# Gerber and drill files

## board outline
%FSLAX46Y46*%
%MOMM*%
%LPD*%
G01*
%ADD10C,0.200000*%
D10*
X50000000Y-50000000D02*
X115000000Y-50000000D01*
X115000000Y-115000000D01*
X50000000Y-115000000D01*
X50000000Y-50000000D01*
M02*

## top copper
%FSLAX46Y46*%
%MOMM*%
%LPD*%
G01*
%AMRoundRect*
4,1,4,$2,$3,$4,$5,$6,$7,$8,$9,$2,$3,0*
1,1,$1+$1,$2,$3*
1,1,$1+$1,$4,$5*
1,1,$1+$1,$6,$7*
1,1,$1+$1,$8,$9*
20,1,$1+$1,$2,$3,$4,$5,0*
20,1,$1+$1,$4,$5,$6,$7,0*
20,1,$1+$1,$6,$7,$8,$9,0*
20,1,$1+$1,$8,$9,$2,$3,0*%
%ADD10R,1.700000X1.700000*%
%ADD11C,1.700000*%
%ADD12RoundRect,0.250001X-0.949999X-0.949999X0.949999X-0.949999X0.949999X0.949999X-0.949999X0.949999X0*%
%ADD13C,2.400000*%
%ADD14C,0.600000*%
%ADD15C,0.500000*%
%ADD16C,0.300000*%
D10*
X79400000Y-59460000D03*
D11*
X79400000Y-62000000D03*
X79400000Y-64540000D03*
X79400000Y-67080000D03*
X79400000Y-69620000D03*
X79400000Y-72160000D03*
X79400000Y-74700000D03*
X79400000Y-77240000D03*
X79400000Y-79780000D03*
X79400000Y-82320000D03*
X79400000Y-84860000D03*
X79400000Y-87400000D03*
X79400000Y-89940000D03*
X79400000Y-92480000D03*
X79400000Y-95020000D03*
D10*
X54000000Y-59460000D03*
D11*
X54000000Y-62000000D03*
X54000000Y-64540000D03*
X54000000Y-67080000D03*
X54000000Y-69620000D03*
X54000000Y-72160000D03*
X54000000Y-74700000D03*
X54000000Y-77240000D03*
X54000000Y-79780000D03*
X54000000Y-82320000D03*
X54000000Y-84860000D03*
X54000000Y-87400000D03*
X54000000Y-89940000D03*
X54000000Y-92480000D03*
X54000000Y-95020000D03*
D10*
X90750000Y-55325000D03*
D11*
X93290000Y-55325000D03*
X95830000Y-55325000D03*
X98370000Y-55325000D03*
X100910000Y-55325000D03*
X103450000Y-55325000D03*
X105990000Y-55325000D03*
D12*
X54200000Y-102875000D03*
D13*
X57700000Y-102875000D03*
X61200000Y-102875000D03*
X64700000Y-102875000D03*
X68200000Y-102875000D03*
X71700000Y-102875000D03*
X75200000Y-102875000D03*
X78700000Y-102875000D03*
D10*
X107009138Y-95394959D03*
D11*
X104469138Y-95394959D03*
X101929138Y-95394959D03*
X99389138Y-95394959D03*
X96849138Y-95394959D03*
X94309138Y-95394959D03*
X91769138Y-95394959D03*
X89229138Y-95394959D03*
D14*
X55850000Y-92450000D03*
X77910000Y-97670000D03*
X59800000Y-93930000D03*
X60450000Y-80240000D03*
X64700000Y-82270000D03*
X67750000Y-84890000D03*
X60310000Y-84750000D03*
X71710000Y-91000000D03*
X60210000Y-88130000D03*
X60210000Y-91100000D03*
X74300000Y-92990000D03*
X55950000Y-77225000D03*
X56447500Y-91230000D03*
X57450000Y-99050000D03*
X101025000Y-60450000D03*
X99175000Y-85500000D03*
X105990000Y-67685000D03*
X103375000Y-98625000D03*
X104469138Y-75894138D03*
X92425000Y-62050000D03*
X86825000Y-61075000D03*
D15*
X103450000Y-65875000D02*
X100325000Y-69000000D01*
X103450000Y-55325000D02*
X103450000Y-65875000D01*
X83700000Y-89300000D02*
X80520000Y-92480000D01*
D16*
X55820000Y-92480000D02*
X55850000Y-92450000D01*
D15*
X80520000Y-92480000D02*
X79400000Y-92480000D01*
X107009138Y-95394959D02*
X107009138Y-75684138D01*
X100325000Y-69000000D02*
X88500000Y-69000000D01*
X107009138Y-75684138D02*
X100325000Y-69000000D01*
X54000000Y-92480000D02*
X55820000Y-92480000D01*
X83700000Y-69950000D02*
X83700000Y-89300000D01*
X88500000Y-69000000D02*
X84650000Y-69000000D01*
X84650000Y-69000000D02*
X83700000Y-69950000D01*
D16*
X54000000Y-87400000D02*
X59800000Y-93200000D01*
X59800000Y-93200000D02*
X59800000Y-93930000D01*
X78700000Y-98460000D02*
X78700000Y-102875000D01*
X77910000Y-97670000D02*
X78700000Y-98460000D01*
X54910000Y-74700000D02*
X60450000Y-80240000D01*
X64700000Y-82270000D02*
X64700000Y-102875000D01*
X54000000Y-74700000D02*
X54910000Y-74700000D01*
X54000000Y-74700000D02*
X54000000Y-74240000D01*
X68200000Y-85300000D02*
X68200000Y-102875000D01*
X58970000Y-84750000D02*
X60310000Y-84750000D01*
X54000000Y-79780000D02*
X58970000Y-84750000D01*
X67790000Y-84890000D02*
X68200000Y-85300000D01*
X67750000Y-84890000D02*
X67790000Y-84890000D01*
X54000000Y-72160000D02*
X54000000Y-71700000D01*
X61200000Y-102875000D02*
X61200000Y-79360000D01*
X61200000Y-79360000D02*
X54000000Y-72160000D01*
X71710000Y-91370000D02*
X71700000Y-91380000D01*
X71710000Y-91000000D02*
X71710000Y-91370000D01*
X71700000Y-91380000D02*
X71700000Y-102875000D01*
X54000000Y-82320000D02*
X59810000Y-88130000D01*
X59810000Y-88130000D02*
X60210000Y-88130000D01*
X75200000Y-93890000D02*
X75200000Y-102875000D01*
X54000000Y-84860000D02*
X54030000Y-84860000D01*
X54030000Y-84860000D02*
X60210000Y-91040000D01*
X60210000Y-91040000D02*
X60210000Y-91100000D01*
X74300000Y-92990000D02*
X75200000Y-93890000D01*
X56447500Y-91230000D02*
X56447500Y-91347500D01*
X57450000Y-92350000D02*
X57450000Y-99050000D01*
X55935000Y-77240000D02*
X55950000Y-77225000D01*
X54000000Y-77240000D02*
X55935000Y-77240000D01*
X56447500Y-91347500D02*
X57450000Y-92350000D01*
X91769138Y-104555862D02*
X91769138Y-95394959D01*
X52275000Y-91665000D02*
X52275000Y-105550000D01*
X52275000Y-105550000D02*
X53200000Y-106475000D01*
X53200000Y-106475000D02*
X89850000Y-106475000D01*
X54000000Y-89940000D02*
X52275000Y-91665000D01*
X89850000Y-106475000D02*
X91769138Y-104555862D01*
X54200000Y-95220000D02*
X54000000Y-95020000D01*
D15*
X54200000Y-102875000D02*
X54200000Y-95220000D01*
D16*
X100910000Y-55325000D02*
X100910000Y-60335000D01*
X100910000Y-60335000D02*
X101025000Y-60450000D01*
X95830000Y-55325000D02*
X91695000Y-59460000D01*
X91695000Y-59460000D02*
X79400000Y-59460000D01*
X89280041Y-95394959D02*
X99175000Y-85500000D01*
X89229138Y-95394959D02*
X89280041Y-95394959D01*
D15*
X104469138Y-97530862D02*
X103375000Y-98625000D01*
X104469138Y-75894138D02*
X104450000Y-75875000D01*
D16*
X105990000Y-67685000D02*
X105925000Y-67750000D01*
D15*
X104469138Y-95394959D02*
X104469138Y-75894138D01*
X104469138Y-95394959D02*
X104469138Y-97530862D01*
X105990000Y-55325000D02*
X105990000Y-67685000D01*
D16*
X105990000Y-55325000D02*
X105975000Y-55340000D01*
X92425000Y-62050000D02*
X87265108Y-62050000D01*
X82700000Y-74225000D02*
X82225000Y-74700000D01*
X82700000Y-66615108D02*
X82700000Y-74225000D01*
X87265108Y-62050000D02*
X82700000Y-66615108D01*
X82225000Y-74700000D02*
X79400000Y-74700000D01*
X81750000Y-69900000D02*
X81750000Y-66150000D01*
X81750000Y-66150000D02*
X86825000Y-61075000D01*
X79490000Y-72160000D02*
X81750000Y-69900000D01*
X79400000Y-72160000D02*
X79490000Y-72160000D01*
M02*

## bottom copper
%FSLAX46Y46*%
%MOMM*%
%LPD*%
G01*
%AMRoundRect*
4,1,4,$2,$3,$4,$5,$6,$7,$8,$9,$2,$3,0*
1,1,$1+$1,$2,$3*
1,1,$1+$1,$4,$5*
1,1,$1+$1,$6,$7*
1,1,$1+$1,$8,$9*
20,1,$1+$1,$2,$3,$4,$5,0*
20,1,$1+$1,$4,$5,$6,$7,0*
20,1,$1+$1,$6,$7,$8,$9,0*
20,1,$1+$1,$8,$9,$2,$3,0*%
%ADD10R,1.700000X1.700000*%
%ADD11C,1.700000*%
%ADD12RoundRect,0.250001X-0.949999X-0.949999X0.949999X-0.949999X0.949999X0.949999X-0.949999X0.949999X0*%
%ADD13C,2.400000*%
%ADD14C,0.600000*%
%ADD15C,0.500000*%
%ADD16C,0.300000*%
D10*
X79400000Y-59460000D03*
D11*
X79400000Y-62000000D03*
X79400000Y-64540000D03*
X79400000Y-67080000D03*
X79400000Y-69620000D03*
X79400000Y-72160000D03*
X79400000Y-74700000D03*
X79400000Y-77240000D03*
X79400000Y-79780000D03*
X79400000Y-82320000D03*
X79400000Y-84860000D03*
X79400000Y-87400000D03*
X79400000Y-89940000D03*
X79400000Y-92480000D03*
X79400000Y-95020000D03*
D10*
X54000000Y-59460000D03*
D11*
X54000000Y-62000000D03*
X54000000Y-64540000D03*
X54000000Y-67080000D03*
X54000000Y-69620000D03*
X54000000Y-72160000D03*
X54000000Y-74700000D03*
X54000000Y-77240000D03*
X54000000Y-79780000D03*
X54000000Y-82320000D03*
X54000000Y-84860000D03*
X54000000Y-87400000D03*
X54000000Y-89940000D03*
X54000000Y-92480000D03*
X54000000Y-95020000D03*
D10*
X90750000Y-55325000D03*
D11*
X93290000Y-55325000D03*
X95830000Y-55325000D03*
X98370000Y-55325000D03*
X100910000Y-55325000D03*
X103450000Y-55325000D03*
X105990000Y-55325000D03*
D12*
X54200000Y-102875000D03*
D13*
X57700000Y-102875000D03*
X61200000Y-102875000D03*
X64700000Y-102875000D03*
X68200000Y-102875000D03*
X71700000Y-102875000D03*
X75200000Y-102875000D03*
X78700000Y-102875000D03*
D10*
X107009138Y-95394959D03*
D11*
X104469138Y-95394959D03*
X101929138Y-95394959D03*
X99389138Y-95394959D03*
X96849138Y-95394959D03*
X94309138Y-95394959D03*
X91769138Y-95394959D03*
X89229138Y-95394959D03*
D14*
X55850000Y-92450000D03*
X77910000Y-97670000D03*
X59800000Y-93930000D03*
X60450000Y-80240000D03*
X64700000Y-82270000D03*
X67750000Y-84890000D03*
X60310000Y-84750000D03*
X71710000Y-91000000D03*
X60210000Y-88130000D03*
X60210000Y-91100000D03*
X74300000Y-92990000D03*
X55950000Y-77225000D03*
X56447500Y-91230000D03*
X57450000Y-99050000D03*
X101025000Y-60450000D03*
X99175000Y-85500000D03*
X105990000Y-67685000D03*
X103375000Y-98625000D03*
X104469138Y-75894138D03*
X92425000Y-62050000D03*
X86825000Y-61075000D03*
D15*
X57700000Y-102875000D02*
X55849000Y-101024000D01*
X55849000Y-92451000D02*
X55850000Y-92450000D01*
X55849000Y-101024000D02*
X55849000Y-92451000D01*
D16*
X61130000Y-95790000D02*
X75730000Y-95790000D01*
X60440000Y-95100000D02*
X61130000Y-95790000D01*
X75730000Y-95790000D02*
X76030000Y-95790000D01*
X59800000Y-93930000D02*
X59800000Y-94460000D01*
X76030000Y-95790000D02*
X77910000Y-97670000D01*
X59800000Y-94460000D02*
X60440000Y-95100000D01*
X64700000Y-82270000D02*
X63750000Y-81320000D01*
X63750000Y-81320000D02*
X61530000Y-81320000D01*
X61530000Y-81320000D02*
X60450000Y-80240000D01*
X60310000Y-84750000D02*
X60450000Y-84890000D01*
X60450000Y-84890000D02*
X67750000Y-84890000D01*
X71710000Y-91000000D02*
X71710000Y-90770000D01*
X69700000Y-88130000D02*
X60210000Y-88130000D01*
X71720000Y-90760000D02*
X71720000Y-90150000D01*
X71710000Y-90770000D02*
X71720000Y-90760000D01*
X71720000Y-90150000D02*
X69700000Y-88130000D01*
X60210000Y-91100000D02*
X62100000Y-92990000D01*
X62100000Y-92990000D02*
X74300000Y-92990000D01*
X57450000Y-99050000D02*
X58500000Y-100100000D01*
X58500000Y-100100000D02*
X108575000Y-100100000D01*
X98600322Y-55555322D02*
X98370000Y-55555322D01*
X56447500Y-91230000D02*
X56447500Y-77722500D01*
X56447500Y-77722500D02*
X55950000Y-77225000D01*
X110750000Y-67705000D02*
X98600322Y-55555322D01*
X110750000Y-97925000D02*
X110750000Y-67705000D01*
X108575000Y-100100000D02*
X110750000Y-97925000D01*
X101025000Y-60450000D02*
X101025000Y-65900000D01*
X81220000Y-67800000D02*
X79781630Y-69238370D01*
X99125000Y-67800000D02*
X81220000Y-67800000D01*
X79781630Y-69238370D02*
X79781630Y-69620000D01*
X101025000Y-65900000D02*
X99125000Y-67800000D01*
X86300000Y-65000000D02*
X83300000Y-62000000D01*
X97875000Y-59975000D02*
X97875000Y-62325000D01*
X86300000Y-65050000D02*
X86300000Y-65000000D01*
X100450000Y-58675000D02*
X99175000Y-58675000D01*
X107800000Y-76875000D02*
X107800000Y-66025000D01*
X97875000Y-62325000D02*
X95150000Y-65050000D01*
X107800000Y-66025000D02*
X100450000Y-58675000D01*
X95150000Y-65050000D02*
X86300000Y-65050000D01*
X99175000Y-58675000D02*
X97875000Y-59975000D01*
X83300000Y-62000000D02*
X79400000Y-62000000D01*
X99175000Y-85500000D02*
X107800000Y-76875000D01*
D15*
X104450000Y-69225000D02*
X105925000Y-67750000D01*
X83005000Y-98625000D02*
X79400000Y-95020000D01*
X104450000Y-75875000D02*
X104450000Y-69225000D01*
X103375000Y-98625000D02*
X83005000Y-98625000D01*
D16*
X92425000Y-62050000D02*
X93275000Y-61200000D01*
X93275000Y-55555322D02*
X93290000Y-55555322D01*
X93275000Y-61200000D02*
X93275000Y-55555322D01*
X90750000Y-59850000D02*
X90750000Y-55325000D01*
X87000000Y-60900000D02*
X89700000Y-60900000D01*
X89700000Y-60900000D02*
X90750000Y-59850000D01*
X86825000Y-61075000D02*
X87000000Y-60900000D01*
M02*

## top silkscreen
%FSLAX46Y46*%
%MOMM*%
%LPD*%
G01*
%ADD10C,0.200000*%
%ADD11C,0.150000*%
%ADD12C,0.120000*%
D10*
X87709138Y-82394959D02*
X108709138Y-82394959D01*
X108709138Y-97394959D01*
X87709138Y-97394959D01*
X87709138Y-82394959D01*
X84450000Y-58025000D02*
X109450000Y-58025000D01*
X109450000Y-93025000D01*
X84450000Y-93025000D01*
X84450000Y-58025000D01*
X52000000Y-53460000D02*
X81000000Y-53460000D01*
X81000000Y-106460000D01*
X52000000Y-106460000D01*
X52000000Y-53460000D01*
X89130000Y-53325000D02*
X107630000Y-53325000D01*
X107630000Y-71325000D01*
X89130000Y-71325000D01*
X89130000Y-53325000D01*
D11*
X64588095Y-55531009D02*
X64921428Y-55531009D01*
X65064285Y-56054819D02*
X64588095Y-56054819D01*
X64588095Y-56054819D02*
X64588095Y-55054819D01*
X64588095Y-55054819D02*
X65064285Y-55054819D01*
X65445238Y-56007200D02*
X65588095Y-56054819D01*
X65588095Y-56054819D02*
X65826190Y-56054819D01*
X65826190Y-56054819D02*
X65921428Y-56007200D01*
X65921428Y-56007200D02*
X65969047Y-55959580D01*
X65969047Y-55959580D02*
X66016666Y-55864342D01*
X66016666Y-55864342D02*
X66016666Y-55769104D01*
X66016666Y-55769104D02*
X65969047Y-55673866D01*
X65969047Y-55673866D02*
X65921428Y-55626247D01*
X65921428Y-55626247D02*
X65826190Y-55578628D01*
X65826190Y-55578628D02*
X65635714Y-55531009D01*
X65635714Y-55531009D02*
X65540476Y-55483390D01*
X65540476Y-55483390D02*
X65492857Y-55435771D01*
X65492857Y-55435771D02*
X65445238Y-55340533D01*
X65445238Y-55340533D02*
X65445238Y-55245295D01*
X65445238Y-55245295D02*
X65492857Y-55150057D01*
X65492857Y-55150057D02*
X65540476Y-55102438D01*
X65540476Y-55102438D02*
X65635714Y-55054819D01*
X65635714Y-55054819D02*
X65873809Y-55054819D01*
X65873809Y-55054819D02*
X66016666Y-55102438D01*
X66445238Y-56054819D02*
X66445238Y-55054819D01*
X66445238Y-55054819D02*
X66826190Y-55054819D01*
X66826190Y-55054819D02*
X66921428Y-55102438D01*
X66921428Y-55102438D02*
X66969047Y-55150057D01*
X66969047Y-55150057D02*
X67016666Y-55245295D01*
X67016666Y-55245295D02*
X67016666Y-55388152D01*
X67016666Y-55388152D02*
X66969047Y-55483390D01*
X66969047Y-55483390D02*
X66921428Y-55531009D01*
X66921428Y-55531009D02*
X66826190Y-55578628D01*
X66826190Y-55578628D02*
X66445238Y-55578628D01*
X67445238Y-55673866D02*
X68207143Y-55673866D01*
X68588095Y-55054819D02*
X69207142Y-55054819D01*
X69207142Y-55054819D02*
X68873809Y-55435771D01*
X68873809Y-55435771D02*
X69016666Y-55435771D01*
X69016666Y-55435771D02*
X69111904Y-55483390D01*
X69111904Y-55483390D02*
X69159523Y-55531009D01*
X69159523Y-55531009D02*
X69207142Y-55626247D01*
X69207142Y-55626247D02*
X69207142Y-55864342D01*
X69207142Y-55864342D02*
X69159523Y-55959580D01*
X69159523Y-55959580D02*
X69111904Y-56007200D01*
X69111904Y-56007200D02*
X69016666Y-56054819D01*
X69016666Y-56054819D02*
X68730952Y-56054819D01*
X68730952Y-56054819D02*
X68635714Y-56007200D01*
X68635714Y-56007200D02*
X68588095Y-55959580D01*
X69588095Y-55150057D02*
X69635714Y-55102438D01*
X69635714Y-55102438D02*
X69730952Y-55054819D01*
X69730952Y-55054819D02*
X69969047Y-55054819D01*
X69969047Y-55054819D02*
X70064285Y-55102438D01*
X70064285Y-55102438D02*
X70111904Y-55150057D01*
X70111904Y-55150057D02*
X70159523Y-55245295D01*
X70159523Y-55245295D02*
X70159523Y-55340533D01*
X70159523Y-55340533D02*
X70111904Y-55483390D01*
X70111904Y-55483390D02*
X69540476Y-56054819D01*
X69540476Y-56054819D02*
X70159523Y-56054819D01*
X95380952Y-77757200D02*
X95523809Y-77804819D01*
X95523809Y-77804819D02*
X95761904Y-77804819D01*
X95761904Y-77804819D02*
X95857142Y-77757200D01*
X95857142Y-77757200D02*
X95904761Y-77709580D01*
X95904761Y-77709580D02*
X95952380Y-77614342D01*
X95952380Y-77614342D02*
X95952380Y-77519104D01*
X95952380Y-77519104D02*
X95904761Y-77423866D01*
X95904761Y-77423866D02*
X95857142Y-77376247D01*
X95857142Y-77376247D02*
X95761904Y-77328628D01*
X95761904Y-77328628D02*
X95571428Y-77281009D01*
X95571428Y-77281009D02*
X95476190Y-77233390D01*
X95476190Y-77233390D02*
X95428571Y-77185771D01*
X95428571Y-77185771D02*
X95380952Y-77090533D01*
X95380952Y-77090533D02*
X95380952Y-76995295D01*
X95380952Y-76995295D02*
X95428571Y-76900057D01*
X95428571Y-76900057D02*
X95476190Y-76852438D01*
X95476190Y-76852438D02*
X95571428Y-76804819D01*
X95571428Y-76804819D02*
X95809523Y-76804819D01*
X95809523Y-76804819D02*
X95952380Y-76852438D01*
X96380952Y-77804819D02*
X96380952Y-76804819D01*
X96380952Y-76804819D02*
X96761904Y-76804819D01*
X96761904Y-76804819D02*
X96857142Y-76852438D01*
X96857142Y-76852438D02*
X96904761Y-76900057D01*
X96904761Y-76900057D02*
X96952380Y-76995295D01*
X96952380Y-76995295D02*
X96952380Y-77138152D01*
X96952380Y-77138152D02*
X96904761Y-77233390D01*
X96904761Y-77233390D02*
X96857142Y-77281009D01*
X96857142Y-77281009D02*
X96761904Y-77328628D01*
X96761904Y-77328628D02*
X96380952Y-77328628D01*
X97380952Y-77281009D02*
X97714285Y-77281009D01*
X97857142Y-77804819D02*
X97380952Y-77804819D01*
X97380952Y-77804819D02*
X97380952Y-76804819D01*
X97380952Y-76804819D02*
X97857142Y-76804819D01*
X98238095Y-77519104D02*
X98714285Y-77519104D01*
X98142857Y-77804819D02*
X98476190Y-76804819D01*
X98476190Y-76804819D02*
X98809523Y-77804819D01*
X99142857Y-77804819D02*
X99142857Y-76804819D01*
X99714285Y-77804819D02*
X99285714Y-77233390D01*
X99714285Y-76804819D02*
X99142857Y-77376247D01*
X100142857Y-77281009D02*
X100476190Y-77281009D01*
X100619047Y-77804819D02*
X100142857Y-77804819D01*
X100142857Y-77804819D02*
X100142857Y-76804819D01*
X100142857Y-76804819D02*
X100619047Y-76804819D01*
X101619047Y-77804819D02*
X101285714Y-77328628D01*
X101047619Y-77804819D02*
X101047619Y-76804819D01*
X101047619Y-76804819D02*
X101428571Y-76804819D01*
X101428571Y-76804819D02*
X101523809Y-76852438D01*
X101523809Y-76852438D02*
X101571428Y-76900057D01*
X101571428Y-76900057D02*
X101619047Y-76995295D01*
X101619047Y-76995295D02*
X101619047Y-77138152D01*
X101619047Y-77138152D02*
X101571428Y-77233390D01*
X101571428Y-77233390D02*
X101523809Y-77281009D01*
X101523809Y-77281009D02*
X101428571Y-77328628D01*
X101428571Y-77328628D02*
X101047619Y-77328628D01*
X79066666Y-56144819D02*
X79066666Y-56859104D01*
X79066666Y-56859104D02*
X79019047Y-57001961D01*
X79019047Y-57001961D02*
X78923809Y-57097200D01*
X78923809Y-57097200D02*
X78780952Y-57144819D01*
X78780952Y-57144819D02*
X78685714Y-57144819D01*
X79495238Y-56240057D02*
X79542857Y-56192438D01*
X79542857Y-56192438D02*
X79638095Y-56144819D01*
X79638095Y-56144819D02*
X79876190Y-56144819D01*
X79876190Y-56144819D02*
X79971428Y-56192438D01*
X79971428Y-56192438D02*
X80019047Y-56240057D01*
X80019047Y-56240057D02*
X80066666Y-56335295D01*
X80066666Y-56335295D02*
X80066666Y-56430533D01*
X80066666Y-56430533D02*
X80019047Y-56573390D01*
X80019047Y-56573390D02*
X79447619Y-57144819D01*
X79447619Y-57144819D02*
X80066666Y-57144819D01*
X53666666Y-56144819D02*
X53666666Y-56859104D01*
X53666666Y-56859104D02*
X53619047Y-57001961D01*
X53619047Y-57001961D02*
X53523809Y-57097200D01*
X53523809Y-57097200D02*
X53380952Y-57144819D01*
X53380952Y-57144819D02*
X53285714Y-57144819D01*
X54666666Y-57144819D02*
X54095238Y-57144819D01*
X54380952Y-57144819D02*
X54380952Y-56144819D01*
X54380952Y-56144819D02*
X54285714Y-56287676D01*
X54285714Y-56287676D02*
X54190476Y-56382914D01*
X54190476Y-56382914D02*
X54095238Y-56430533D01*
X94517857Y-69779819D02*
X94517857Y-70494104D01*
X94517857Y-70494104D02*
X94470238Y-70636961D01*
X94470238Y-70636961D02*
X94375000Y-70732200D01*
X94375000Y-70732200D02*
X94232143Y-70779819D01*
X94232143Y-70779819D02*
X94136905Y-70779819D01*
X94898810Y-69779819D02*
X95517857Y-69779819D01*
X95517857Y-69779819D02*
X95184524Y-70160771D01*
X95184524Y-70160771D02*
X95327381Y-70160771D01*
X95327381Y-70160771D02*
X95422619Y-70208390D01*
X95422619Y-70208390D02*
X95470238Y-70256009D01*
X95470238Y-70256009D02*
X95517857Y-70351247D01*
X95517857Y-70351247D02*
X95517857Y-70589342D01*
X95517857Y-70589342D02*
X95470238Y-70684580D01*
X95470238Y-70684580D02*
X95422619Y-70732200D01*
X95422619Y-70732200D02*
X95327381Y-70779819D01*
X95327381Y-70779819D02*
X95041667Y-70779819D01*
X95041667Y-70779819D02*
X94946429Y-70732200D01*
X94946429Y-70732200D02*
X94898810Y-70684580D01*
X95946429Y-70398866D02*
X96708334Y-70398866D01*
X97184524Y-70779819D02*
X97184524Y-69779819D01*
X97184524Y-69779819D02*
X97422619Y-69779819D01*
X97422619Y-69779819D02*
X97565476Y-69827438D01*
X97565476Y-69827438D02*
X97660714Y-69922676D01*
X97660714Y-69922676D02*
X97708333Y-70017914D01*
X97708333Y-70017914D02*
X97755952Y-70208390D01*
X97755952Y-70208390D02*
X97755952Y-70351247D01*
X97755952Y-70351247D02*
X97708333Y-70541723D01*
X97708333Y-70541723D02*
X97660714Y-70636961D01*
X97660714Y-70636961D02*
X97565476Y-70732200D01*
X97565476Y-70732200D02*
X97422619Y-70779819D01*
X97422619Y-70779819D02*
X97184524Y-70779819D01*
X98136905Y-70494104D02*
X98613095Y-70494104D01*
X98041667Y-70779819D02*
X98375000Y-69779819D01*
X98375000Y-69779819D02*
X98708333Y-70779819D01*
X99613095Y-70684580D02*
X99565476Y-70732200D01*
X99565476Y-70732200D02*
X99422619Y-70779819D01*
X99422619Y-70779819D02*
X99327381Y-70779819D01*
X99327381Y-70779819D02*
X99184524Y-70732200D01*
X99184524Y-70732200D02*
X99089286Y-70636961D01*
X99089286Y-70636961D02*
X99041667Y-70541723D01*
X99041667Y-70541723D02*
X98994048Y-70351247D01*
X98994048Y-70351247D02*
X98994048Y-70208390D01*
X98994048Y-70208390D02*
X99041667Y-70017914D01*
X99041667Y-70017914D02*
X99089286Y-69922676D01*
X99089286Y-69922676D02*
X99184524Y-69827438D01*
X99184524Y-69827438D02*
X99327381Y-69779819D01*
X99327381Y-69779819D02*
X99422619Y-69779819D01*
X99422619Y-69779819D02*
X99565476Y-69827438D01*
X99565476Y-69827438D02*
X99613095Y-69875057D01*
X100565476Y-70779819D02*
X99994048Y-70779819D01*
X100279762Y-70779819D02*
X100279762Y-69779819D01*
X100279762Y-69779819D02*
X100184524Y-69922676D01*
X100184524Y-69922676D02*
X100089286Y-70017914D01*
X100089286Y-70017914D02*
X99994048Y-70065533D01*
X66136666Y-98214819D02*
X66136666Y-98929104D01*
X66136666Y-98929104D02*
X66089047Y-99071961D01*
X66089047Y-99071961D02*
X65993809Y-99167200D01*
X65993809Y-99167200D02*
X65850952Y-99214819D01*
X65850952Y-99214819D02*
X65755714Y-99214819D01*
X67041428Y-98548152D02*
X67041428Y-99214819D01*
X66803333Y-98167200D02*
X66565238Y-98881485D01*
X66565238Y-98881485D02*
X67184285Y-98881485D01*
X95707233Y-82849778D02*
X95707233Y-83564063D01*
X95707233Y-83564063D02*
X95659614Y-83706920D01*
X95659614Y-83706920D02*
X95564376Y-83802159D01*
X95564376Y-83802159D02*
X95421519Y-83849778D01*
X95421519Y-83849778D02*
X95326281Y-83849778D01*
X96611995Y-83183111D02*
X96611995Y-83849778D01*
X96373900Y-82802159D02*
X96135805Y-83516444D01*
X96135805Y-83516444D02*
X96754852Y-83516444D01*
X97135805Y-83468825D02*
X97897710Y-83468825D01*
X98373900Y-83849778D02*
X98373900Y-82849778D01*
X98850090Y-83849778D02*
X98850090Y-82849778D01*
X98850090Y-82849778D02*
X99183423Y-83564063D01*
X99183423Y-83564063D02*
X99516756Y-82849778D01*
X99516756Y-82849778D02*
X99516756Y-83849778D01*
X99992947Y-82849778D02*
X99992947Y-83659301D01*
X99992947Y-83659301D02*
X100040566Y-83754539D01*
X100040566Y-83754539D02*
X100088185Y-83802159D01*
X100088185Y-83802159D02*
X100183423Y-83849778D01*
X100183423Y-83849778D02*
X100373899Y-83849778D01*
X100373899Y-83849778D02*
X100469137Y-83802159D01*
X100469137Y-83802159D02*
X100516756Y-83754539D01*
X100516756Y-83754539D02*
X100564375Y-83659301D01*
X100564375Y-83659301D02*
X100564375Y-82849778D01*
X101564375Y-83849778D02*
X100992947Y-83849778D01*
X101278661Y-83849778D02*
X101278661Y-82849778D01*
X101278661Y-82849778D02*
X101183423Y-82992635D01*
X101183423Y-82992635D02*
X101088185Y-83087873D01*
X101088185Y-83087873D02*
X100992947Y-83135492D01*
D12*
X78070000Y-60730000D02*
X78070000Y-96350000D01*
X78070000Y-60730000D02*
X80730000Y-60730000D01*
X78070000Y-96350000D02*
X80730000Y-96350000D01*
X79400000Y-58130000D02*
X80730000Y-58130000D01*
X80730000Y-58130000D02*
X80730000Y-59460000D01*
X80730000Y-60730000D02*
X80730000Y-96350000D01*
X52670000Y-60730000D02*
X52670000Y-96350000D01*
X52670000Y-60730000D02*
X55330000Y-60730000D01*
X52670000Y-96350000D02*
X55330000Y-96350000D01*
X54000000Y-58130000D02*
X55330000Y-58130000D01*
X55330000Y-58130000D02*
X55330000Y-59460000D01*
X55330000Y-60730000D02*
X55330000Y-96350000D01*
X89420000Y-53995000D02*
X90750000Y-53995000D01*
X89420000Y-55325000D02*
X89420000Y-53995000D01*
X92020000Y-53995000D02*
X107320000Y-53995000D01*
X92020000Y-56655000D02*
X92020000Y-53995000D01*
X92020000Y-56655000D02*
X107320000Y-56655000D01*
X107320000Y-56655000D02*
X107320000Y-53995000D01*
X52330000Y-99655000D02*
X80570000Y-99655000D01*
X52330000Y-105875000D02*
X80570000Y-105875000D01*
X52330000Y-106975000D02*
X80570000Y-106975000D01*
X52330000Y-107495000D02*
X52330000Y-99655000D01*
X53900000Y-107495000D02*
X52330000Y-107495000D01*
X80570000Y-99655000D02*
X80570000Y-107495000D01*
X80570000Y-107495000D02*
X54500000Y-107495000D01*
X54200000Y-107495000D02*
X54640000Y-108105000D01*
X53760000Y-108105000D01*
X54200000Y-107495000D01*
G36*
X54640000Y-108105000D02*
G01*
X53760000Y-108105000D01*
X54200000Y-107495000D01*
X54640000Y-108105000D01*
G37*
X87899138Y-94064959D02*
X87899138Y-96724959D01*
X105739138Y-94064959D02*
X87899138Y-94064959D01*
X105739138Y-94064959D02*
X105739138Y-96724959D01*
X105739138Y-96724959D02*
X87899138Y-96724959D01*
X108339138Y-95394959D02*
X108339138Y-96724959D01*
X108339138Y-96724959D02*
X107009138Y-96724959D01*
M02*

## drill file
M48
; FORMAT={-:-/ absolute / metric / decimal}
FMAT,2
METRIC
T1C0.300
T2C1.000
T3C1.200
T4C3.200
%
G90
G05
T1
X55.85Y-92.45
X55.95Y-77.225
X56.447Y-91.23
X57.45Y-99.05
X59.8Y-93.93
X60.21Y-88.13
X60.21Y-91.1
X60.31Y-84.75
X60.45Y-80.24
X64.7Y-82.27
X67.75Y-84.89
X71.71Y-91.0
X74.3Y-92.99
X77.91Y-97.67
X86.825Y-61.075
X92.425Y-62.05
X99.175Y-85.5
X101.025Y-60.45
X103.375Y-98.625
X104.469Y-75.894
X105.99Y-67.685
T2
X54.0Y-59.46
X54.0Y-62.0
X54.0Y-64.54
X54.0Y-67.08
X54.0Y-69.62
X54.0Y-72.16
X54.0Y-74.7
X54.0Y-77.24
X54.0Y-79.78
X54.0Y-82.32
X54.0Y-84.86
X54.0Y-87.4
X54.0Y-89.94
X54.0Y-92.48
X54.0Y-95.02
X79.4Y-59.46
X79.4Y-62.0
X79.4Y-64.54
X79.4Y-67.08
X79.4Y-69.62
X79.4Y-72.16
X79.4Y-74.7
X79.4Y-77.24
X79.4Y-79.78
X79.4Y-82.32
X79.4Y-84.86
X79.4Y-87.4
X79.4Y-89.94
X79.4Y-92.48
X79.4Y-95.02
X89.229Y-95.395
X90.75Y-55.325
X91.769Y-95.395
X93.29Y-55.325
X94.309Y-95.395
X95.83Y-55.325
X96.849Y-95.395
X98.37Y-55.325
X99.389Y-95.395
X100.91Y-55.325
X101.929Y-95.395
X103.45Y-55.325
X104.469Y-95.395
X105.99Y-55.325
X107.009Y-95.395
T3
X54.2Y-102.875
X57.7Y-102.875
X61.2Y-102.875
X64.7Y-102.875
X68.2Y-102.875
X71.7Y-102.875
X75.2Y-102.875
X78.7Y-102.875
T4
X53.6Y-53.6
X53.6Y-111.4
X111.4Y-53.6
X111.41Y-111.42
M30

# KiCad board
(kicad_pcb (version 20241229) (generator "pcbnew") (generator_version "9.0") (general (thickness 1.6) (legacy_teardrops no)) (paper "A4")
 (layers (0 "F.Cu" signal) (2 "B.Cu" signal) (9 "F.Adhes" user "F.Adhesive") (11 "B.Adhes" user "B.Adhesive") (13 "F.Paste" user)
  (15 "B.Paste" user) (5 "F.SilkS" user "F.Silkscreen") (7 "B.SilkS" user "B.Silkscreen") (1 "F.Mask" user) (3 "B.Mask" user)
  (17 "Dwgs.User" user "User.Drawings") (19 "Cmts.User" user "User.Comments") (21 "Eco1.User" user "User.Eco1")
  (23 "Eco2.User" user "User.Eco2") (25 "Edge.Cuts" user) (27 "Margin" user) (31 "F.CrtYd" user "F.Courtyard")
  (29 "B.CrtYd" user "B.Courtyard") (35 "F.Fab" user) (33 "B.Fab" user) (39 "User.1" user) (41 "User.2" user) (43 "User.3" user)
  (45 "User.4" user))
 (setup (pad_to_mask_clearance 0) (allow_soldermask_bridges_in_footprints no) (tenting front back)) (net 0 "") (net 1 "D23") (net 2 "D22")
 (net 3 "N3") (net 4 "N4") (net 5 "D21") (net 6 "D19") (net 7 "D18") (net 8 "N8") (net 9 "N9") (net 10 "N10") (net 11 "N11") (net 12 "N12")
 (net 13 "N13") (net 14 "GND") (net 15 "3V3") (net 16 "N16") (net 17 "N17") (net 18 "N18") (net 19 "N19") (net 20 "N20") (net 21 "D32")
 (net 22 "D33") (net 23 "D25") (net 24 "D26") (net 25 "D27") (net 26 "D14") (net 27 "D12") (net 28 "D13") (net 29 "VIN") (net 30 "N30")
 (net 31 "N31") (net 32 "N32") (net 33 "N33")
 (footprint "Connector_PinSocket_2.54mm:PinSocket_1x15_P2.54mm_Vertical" (layer "F.Cu") (at 79.4 59.46)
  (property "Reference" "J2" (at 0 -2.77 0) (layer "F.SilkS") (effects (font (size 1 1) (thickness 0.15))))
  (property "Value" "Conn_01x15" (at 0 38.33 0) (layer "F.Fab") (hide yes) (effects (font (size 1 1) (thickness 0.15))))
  (fp_line (start -1.33 1.27) (end -1.33 36.89) (stroke (width 0.12) (type solid)) (layer "F.SilkS"))
  (fp_line (start -1.33 1.27) (end 1.33 1.27) (stroke (width 0.12) (type solid)) (layer "F.SilkS"))
  (fp_line (start -1.33 36.89) (end 1.33 36.89) (stroke (width 0.12) (type solid)) (layer "F.SilkS"))
  (fp_line (start 0 -1.33) (end 1.33 -1.33) (stroke (width 0.12) (type solid)) (layer "F.SilkS"))
  (fp_line (start 1.33 -1.33) (end 1.33 0) (stroke (width 0.12) (type solid)) (layer "F.SilkS"))
  (fp_line (start 1.33 1.27) (end 1.33 36.89) (stroke (width 0.12) (type solid)) (layer "F.SilkS"))
  (pad "1" thru_hole rect (at 0 0) (size 1.7 1.7) (drill 1) (layers "*.Cu" "*.Mask") (remove_unused_layers no) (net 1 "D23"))
  (pad "2" thru_hole circle (at 0 2.54) (size 1.7 1.7) (drill 1) (layers "*.Cu" "*.Mask") (remove_unused_layers no) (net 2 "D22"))
  (pad "3" thru_hole circle (at 0 5.08) (size 1.7 1.7) (drill 1) (layers "*.Cu" "*.Mask") (remove_unused_layers no) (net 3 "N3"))
  (pad "4" thru_hole circle (at 0 7.62) (size 1.7 1.7) (drill 1) (layers "*.Cu" "*.Mask") (remove_unused_layers no) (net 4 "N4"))
  (pad "5" thru_hole circle (at 0 10.16) (size 1.7 1.7) (drill 1) (layers "*.Cu" "*.Mask") (remove_unused_layers no) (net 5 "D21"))
  (pad "6" thru_hole circle (at 0 12.7) (size 1.7 1.7) (drill 1) (layers "*.Cu" "*.Mask") (remove_unused_layers no) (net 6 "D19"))
  (pad "7" thru_hole circle (at 0 15.24) (size 1.7 1.7) (drill 1) (layers "*.Cu" "*.Mask") (remove_unused_layers no) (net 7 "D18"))
  (pad "8" thru_hole circle (at 0 17.78) (size 1.7 1.7) (drill 1) (layers "*.Cu" "*.Mask") (remove_unused_layers no) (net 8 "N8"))
  (pad "9" thru_hole circle (at 0 20.32) (size 1.7 1.7) (drill 1) (layers "*.Cu" "*.Mask") (remove_unused_layers no) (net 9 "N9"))
  (pad "10" thru_hole circle (at 0 22.86) (size 1.7 1.7) (drill 1) (layers "*.Cu" "*.Mask") (remove_unused_layers no) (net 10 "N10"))
  (pad "11" thru_hole circle (at 0 25.4) (size 1.7 1.7) (drill 1) (layers "*.Cu" "*.Mask") (remove_unused_layers no) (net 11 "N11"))
  (pad "12" thru_hole circle (at 0 27.94) (size 1.7 1.7) (drill 1) (layers "*.Cu" "*.Mask") (remove_unused_layers no) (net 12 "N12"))
  (pad "13" thru_hole circle (at 0 30.48) (size 1.7 1.7) (drill 1) (layers "*.Cu" "*.Mask") (remove_unused_layers no) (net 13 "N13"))
  (pad "14" thru_hole circle (at 0 33.02) (size 1.7 1.7) (drill 1) (layers "*.Cu" "*.Mask") (remove_unused_layers no) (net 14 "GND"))
  (pad "15" thru_hole circle (at 0 35.56) (size 1.7 1.7) (drill 1) (layers "*.Cu" "*.Mask") (remove_unused_layers no) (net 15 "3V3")))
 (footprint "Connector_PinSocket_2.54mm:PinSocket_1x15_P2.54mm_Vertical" (layer "F.Cu") (at 54 59.46)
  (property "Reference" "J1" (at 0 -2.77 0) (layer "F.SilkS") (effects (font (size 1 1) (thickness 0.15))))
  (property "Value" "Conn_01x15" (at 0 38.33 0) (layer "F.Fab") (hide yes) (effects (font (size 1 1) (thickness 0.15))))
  (fp_line (start -1.33 1.27) (end -1.33 36.89) (stroke (width 0.12) (type solid)) (layer "F.SilkS"))
  (fp_line (start -1.33 1.27) (end 1.33 1.27) (stroke (width 0.12) (type solid)) (layer "F.SilkS"))
  (fp_line (start -1.33 36.89) (end 1.33 36.89) (stroke (width 0.12) (type solid)) (layer "F.SilkS"))
  (fp_line (start 0 -1.33) (end 1.33 -1.33) (stroke (width 0.12) (type solid)) (layer "F.SilkS"))
  (fp_line (start 1.33 -1.33) (end 1.33 0) (stroke (width 0.12) (type solid)) (layer "F.SilkS"))
  (fp_line (start 1.33 1.27) (end 1.33 36.89) (stroke (width 0.12) (type solid)) (layer "F.SilkS"))
  (pad "1" thru_hole rect (at 0 0) (size 1.7 1.7) (drill 1) (layers "*.Cu" "*.Mask") (remove_unused_layers no) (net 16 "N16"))
  (pad "2" thru_hole circle (at 0 2.54) (size 1.7 1.7) (drill 1) (layers "*.Cu" "*.Mask") (remove_unused_layers no) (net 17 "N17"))
  (pad "3" thru_hole circle (at 0 5.08) (size 1.7 1.7) (drill 1) (layers "*.Cu" "*.Mask") (remove_unused_layers no) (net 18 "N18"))
  (pad "4" thru_hole circle (at 0 7.62) (size 1.7 1.7) (drill 1) (layers "*.Cu" "*.Mask") (remove_unused_layers no) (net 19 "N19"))
  (pad "5" thru_hole circle (at 0 10.16) (size 1.7 1.7) (drill 1) (layers "*.Cu" "*.Mask") (remove_unused_layers no) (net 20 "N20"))
  (pad "6" thru_hole circle (at 0 12.7) (size 1.7 1.7) (drill 1) (layers "*.Cu" "*.Mask") (remove_unused_layers no) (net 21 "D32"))
  (pad "7" thru_hole circle (at 0 15.24) (size 1.7 1.7) (drill 1) (layers "*.Cu" "*.Mask") (remove_unused_layers no) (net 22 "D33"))
  (pad "8" thru_hole circle (at 0 17.78) (size 1.7 1.7) (drill 1) (layers "*.Cu" "*.Mask") (remove_unused_layers no) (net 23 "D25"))
  (pad "9" thru_hole circle (at 0 20.32) (size 1.7 1.7) (drill 1) (layers "*.Cu" "*.Mask") (remove_unused_layers no) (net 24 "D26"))
  (pad "10" thru_hole circle (at 0 22.86) (size 1.7 1.7) (drill 1) (layers "*.Cu" "*.Mask") (remove_unused_layers no) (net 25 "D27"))
  (pad "11" thru_hole circle (at 0 25.4) (size 1.7 1.7) (drill 1) (layers "*.Cu" "*.Mask") (remove_unused_layers no) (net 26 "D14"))
  (pad "12" thru_hole circle (at 0 27.94) (size 1.7 1.7) (drill 1) (layers "*.Cu" "*.Mask") (remove_unused_layers no) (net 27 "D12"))
  (pad "13" thru_hole circle (at 0 30.48) (size 1.7 1.7) (drill 1) (layers "*.Cu" "*.Mask") (remove_unused_layers no) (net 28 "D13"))
  (pad "14" thru_hole circle (at 0 33.02) (size 1.7 1.7) (drill 1) (layers "*.Cu" "*.Mask") (remove_unused_layers no) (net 14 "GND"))
  (pad "15" thru_hole circle (at 0 35.56) (size 1.7 1.7) (drill 1) (layers "*.Cu" "*.Mask") (remove_unused_layers no) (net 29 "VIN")))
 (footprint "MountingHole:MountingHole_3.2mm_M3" (layer "F.Cu") (at 53.6 53.6)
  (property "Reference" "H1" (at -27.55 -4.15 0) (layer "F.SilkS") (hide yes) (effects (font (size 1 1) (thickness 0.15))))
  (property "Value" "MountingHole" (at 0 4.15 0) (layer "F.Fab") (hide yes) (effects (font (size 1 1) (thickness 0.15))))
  (pad "" np_thru_hole circle (at 0 0) (size 3.2 3.2) (drill 3.2) (layers "*.Cu" "*.Mask")))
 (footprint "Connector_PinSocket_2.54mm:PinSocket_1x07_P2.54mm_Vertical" (layer "F.Cu") (at 90.75 55.325 90)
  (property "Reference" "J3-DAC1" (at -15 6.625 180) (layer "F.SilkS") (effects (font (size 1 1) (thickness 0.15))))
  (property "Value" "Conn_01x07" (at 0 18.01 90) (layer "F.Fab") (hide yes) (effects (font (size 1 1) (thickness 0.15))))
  (fp_line (start 1.33 -1.33) (end 1.33 0) (stroke (width 0.12) (type solid)) (layer "F.SilkS"))
  (fp_line (start 0 -1.33) (end 1.33 -1.33) (stroke (width 0.12) (type solid)) (layer "F.SilkS"))
  (fp_line (start 1.33 1.27) (end 1.33 16.57) (stroke (width 0.12) (type solid)) (layer "F.SilkS"))
  (fp_line (start -1.33 1.27) (end 1.33 1.27) (stroke (width 0.12) (type solid)) (layer "F.SilkS"))
  (fp_line (start -1.33 1.27) (end -1.33 16.57) (stroke (width 0.12) (type solid)) (layer "F.SilkS"))
  (fp_line (start -1.33 16.57) (end 1.33 16.57) (stroke (width 0.12) (type solid)) (layer "F.SilkS"))
  (pad "1" thru_hole rect (at 0 0 90) (size 1.7 1.7) (drill 1) (layers "*.Cu" "*.Mask") (remove_unused_layers no) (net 6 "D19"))
  (pad "2" thru_hole circle (at 0 2.54 90) (size 1.7 1.7) (drill 1) (layers "*.Cu" "*.Mask") (remove_unused_layers no) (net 7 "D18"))
  (pad "3" thru_hole circle (at 0 5.08 90) (size 1.7 1.7) (drill 1) (layers "*.Cu" "*.Mask") (remove_unused_layers no) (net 1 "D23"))
  (pad "4" thru_hole circle (at 0 7.62 90) (size 1.7 1.7) (drill 1) (layers "*.Cu" "*.Mask") (remove_unused_layers no) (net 23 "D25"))
  (pad "5" thru_hole circle (at 0 10.16 90) (size 1.7 1.7) (drill 1) (layers "*.Cu" "*.Mask") (remove_unused_layers no) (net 5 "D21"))
  (pad "6" thru_hole circle (at 0 12.7 90) (size 1.7 1.7) (drill 1) (layers "*.Cu" "*.Mask") (remove_unused_layers no) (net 14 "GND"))
  (pad "7" thru_hole circle (at 0 15.24 90) (size 1.7 1.7) (drill 1) (layers "*.Cu" "*.Mask") (remove_unused_layers no) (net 15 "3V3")))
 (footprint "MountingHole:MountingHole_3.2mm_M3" (layer "F.Cu") (at 53.6 111.4)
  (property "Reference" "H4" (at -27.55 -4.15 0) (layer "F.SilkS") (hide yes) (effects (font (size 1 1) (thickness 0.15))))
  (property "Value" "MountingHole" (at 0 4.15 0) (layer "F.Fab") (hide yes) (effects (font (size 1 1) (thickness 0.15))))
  (pad "" np_thru_hole circle (at 0 0) (size 3.2 3.2) (drill 3.2) (layers "*.Cu" "*.Mask")))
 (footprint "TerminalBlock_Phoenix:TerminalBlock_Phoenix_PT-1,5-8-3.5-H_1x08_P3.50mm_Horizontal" (layer "F.Cu") (at 54.2 102.875)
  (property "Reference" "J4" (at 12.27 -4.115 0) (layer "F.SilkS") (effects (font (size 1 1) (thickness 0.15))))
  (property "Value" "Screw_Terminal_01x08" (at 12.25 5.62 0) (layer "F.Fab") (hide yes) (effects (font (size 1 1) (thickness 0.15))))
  (fp_line (start -1.87 -3.22) (end 26.37 -3.22) (stroke (width 0.12) (type solid)) (layer "F.SilkS"))
  (fp_line (start -1.87 3) (end 26.37 3) (stroke (width 0.12) (type solid)) (layer "F.SilkS"))
  (fp_line (start -1.87 4.1) (end 26.37 4.1) (stroke (width 0.12) (type solid)) (layer "F.SilkS"))
  (fp_line (start -1.87 4.62) (end -1.87 -3.22) (stroke (width 0.12) (type solid)) (layer "F.SilkS"))
  (fp_line (start -0.3 4.62) (end -1.87 4.62) (stroke (width 0.12) (type solid)) (layer "F.SilkS"))
  (fp_line (start 26.37 -3.22) (end 26.37 4.62) (stroke (width 0.12) (type solid)) (layer "F.SilkS"))
  (fp_line (start 26.37 4.62) (end 0.3 4.62) (stroke (width 0.12) (type solid)) (layer "F.SilkS"))
  (fp_poly (pts (xy 0 4.62) (xy 0.44 5.23) (xy -0.44 5.23)) (stroke (width 0.12) (type solid)) (fill yes) (layer "F.SilkS"))
  (pad "1" thru_hole roundrect (at 0 0) (size 2.4 2.4) (drill 1.2) (layers "*.Cu" "*.Mask") (remove_unused_layers no)
   (roundrect_rratio 0.104167) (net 29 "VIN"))
  (pad "2" thru_hole circle (at 3.5 0) (size 2.4 2.4) (drill 1.2) (layers "*.Cu" "*.Mask") (remove_unused_layers no) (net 14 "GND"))
  (pad "3" thru_hole circle (at 7 0) (size 2.4 2.4) (drill 1.2) (layers "*.Cu" "*.Mask") (remove_unused_layers no) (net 21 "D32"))
  (pad "4" thru_hole circle (at 10.5 0) (size 2.4 2.4) (drill 1.2) (layers "*.Cu" "*.Mask") (remove_unused_layers no) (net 22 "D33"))
  (pad "5" thru_hole circle (at 14 0) (size 2.4 2.4) (drill 1.2) (layers "*.Cu" "*.Mask") (remove_unused_layers no) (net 24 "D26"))
  (pad "6" thru_hole circle (at 17.5 0) (size 2.4 2.4) (drill 1.2) (layers "*.Cu" "*.Mask") (remove_unused_layers no) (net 25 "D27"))
  (pad "7" thru_hole circle (at 21 0) (size 2.4 2.4) (drill 1.2) (layers "*.Cu" "*.Mask") (remove_unused_layers no) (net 26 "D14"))
  (pad "8" thru_hole circle (at 24.5 0) (size 2.4 2.4) (drill 1.2) (layers "*.Cu" "*.Mask") (remove_unused_layers no) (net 27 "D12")))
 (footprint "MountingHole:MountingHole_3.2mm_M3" (layer "F.Cu") (at 111.41 111.42)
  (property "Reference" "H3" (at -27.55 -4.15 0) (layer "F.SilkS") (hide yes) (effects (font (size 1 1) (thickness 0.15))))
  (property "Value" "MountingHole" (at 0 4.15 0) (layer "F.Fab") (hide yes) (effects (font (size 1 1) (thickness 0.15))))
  (pad "" np_thru_hole circle (at 0 0) (size 3.2 3.2) (drill 3.2) (layers "*.Cu" "*.Mask")))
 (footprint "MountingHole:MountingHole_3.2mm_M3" (layer "F.Cu") (at 111.4 53.6)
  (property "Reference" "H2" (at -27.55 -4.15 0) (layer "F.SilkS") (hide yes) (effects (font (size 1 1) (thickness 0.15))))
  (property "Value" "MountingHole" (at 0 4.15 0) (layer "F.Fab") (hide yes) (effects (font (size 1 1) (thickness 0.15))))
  (pad "" np_thru_hole circle (at 0 0) (size 3.2 3.2) (drill 3.2) (layers "*.Cu" "*.Mask")))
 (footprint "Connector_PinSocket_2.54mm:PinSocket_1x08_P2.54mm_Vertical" (layer "F.Cu") (at 107.009138 95.394959 -90)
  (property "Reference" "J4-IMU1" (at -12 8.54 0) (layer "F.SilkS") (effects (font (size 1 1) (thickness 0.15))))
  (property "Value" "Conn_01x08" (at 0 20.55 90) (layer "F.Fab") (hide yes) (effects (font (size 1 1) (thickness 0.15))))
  (fp_line (start -1.33 19.11) (end 1.33 19.11) (stroke (width 0.12) (type solid)) (layer "F.SilkS"))
  (fp_line (start -1.33 1.27) (end -1.33 19.11) (stroke (width 0.12) (type solid)) (layer "F.SilkS"))
  (fp_line (start -1.33 1.27) (end 1.33 1.27) (stroke (width 0.12) (type solid)) (layer "F.SilkS"))
  (fp_line (start 1.33 1.27) (end 1.33 19.11) (stroke (width 0.12) (type solid)) (layer "F.SilkS"))
  (fp_line (start 0 -1.33) (end 1.33 -1.33) (stroke (width 0.12) (type solid)) (layer "F.SilkS"))
  (fp_line (start 1.33 -1.33) (end 1.33 0) (stroke (width 0.12) (type solid)) (layer "F.SilkS"))
  (pad "1" thru_hole rect (at 0 0 270) (size 1.7 1.7) (drill 1) (layers "*.Cu" "*.Mask") (remove_unused_layers no) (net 14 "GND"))
  (pad "2" thru_hole circle (at 0 2.54 270) (size 1.7 1.7) (drill 1) (layers "*.Cu" "*.Mask") (remove_unused_layers no) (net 15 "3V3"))
  (pad "3" thru_hole circle (at 0 5.08 270) (size 1.7 1.7) (drill 1) (layers "*.Cu" "*.Mask") (remove_unused_layers no) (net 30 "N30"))
  (pad "4" thru_hole circle (at 0 7.62 270) (size 1.7 1.7) (drill 1) (layers "*.Cu" "*.Mask") (remove_unused_layers no) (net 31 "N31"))
  (pad "5" thru_hole circle (at 0 10.16 270) (size 1.7 1.7) (drill 1) (layers "*.Cu" "*.Mask") (remove_unused_layers no) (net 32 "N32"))
  (pad "6" thru_hole circle (at 0 12.7 270) (size 1.7 1.7) (drill 1) (layers "*.Cu" "*.Mask") (remove_unused_layers no) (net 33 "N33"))
  (pad "7" thru_hole circle (at 0 15.24 270) (size 1.7 1.7) (drill 1) (layers "*.Cu" "*.Mask") (remove_unused_layers no) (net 28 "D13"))
  (pad "8" thru_hole circle (at 0 17.78 270) (size 1.7 1.7) (drill 1) (layers "*.Cu" "*.Mask") (remove_unused_layers no) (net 2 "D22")))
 (gr_rect (start 87.709138 82.394959) (end 108.709138 97.394959) (stroke (width 0.2) (type solid)) (fill no) (layer "F.SilkS"))
 (gr_rect (start 84.45 58.025) (end 109.45 93.025) (stroke (width 0.2) (type solid)) (fill no) (layer "F.SilkS"))
 (gr_rect (start 52 53.46) (end 81 106.46) (stroke (width 0.2) (type solid)) (fill no) (layer "F.SilkS"))
 (gr_rect (start 89.13 53.325) (end 107.63 71.325) (stroke (width 0.2) (type solid)) (fill no) (layer "F.SilkS"))
 (gr_rect (start 50 50) (end 115 115) (stroke (width 0.2) (type solid)) (fill no) (layer "Edge.Cuts"))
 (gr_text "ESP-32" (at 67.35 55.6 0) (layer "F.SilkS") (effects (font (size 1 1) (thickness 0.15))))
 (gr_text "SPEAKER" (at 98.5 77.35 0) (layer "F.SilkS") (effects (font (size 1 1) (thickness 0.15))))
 (segment (start 103.45 65.875) (end 100.325 69) (width 0.5) (layer "F.Cu") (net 14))
 (segment (start 103.45 55.325) (end 103.45 65.875) (width 0.5) (layer "F.Cu") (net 14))
 (segment (start 83.7 89.3) (end 80.52 92.48) (width 0.5) (layer "F.Cu") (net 14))
 (segment (start 55.82 92.48) (end 55.85 92.45) (width 0.3) (layer "F.Cu") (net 14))
 (segment (start 80.52 92.48) (end 79.4 92.48) (width 0.5) (layer "F.Cu") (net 14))
 (segment (start 107.009138 95.394959) (end 107.009138 75.684138) (width 0.5) (layer "F.Cu") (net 14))
 (segment (start 100.325 69) (end 88.5 69) (width 0.5) (layer "F.Cu") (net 14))
 (segment (start 107.009138 75.684138) (end 100.325 69) (width 0.5) (layer "F.Cu") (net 14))
 (segment (start 54 92.48) (end 55.82 92.48) (width 0.5) (layer "F.Cu") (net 14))
 (segment (start 83.7 69.95) (end 83.7 89.3) (width 0.5) (layer "F.Cu") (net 14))
 (segment (start 88.5 69) (end 84.65 69) (width 0.5) (layer "F.Cu") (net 14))
 (segment (start 84.65 69) (end 83.7 69.95) (width 0.5) (layer "F.Cu") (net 14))
 (via (at 55.85 92.45) (size 0.6) (drill 0.3) (layers "F.Cu" "B.Cu") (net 14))
 (segment (start 57.7 102.875) (end 55.849 101.024) (width 0.5) (layer "B.Cu") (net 14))
 (segment (start 55.849 92.451) (end 55.85 92.45) (width 0.5) (layer "B.Cu") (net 14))
 (segment (start 55.849 101.024) (end 55.849 92.451) (width 0.5) (layer "B.Cu") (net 14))
 (segment (start 54 87.4) (end 59.8 93.2) (width 0.3) (layer "F.Cu") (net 27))
 (segment (start 59.8 93.2) (end 59.8 93.93) (width 0.3) (layer "F.Cu") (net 27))
 (segment (start 78.7 98.46) (end 78.7 102.875) (width 0.3) (layer "F.Cu") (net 27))
 (segment (start 77.91 97.67) (end 78.7 98.46) (width 0.3) (layer "F.Cu") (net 27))
 (via (at 77.91 97.67) (size 0.6) (drill 0.3) (layers "F.Cu" "B.Cu") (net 27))
 (via (at 59.8 93.93) (size 0.6) (drill 0.3) (layers "F.Cu" "B.Cu") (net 27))
 (segment (start 61.13 95.79) (end 75.73 95.79) (width 0.3) (layer "B.Cu") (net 27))
 (segment (start 60.44 95.1) (end 61.13 95.79) (width 0.3) (layer "B.Cu") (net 27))
 (segment (start 75.73 95.79) (end 76.03 95.79) (width 0.3) (layer "B.Cu") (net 27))
 (segment (start 59.8 93.93) (end 59.8 94.46) (width 0.3) (layer "B.Cu") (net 27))
 (segment (start 76.03 95.79) (end 77.91 97.67) (width 0.3) (layer "B.Cu") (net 27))
 (segment (start 59.8 94.46) (end 60.44 95.1) (width 0.3) (layer "B.Cu") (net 27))
 (segment (start 54.91 74.7) (end 60.45 80.24) (width 0.3) (layer "F.Cu") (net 22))
 (segment (start 64.7 82.27) (end 64.7 102.875) (width 0.3) (layer "F.Cu") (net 22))
 (segment (start 54 74.7) (end 54.91 74.7) (width 0.3) (layer "F.Cu") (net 22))
 (segment (start 54 74.7) (end 54 74.24) (width 0.3) (layer "F.Cu") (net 22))
 (via (at 60.45 80.24) (size 0.6) (drill 0.3) (layers "F.Cu" "B.Cu") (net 22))
 (via (at 64.7 82.27) (size 0.6) (drill 0.3) (layers "F.Cu" "B.Cu") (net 22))
 (segment (start 64.7 82.27) (end 63.75 81.32) (width 0.3) (layer "B.Cu") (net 22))
 (segment (start 63.75 81.32) (end 61.53 81.32) (width 0.3) (layer "B.Cu") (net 22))
 (segment (start 61.53 81.32) (end 60.45 80.24) (width 0.3) (layer "B.Cu") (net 22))
 (segment (start 68.2 85.3) (end 68.2 102.875) (width 0.3) (layer "F.Cu") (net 24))
 (segment (start 58.97 84.75) (end 60.31 84.75) (width 0.3) (layer "F.Cu") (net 24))
 (segment (start 54 79.78) (end 58.97 84.75) (width 0.3) (layer "F.Cu") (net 24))
 (segment (start 67.79 84.89) (end 68.2 85.3) (width 0.3) (layer "F.Cu") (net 24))
 (segment (start 67.75 84.89) (end 67.79 84.89) (width 0.3) (layer "F.Cu") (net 24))
 (via (at 67.75 84.89) (size 0.6) (drill 0.3) (layers "F.Cu" "B.Cu") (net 24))
 (via (at 60.31 84.75) (size 0.6) (drill 0.3) (layers "F.Cu" "B.Cu") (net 24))
 (segment (start 60.31 84.75) (end 60.45 84.89) (width 0.3) (layer "B.Cu") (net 24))
 (segment (start 60.45 84.89) (end 67.75 84.89) (width 0.3) (layer "B.Cu") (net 24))
 (segment (start 54 72.16) (end 54 71.7) (width 0.3) (layer "F.Cu") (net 21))
 (segment (start 61.2 102.875) (end 61.2 79.36) (width 0.3) (layer "F.Cu") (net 21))
 (segment (start 61.2 79.36) (end 54 72.16) (width 0.3) (layer "F.Cu") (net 21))
 (segment (start 71.71 91.37) (end 71.7 91.38) (width 0.3) (layer "F.Cu") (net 25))
 (segment (start 71.71 91) (end 71.71 91.37) (width 0.3) (layer "F.Cu") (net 25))
 (segment (start 71.7 91.38) (end 71.7 102.875) (width 0.3) (layer "F.Cu") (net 25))
 (segment (start 54 82.32) (end 59.81 88.13) (width 0.3) (layer "F.Cu") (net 25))
 (segment (start 59.81 88.13) (end 60.21 88.13) (width 0.3) (layer "F.Cu") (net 25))
 (via (at 71.71 91) (size 0.6) (drill 0.3) (layers "F.Cu" "B.Cu") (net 25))
 (via (at 60.21 88.13) (size 0.6) (drill 0.3) (layers "F.Cu" "B.Cu") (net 25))
 (segment (start 71.71 91) (end 71.71 90.77) (width 0.3) (layer "B.Cu") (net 25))
 (segment (start 69.7 88.13) (end 60.21 88.13) (width 0.3) (layer "B.Cu") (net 25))
 (segment (start 71.72 90.76) (end 71.72 90.15) (width 0.3) (layer "B.Cu") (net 25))
 (segment (start 71.71 90.77) (end 71.72 90.76) (width 0.3) (layer "B.Cu") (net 25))
 (segment (start 71.72 90.15) (end 69.7 88.13) (width 0.3) (layer "B.Cu") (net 25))
 (segment (start 75.2 93.89) (end 75.2 102.875) (width 0.3) (layer "F.Cu") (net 26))
 (segment (start 54 84.86) (end 54.03 84.86) (width 0.3) (layer "F.Cu") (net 26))
 (segment (start 54.03 84.86) (end 60.21 91.04) (width 0.3) (layer "F.Cu") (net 26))
 (segment (start 60.21 91.04) (end 60.21 91.1) (width 0.3) (layer "F.Cu") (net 26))
 (segment (start 74.3 92.99) (end 75.2 93.89) (width 0.3) (layer "F.Cu") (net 26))
 (via (at 60.21 91.1) (size 0.6) (drill 0.3) (layers "F.Cu" "B.Cu") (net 26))
 (via (at 74.3 92.99) (size 0.6) (drill 0.3) (layers "F.Cu" "B.Cu") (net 26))
 (segment (start 60.21 91.1) (end 62.1 92.99) (width 0.3) (layer "B.Cu") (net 26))
 (segment (start 62.1 92.99) (end 74.3 92.99) (width 0.3) (layer "B.Cu") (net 26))
 (segment (start 56.4475 91.23) (end 56.4475 91.3475) (width 0.3) (layer "F.Cu") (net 23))
 (segment (start 57.45 92.35) (end 57.45 99.05) (width 0.3) (layer "F.Cu") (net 23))
 (segment (start 55.935 77.24) (end 55.95 77.225) (width 0.3) (layer "F.Cu") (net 23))
 (segment (start 54 77.24) (end 55.935 77.24) (width 0.3) (layer "F.Cu") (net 23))
 (segment (start 56.4475 91.3475) (end 57.45 92.35) (width 0.3) (layer "F.Cu") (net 23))
 (via (at 55.95 77.225) (size 0.6) (drill 0.3) (layers "F.Cu" "B.Cu") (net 23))
 (via (at 56.4475 91.23) (size 0.6) (drill 0.3) (layers "F.Cu" "B.Cu") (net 23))
 (via (at 57.45 99.05) (size 0.6) (drill 0.3) (layers "F.Cu" "B.Cu") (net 23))
 (segment (start 57.45 99.05) (end 58.5 100.1) (width 0.3) (layer "B.Cu") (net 23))
 (segment (start 58.5 100.1) (end 108.575 100.1) (width 0.3) (layer "B.Cu") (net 23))
 (segment (start 98.600322 55.555322) (end 98.37 55.555322) (width 0.3) (layer "B.Cu") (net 23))
 (segment (start 56.4475 91.23) (end 56.4475 77.7225) (width 0.3) (layer "B.Cu") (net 23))
 (segment (start 56.4475 77.7225) (end 55.95 77.225) (width 0.3) (layer "B.Cu") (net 23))
 (segment (start 110.75 67.705) (end 98.600322 55.555322) (width 0.3) (layer "B.Cu") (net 23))
 (segment (start 110.75 97.925) (end 110.75 67.705) (width 0.3) (layer "B.Cu") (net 23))
 (segment (start 108.575 100.1) (end 110.75 97.925) (width 0.3) (layer "B.Cu") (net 23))
 (segment (start 91.769138 104.555862) (end 91.769138 95.394959) (width 0.3) (layer "F.Cu") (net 28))
 (segment (start 52.275 91.665) (end 52.275 105.55) (width 0.3) (layer "F.Cu") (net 28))
 (segment (start 52.275 105.55) (end 53.2 106.475) (width 0.3) (layer "F.Cu") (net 28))
 (segment (start 53.2 106.475) (end 89.85 106.475) (width 0.3) (layer "F.Cu") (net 28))
 (segment (start 54 89.94) (end 52.275 91.665) (width 0.3) (layer "F.Cu") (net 28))
 (segment (start 89.85 106.475) (end 91.769138 104.555862) (width 0.3) (layer "F.Cu") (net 28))
 (segment (start 54.2 95.22) (end 54 95.02) (width 0.3) (layer "F.Cu") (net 29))
 (segment (start 54.2 102.875) (end 54.2 95.22) (width 0.5) (layer "F.Cu") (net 29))
 (segment (start 100.91 55.325) (end 100.91 60.335) (width 0.3) (layer "F.Cu") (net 5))
 (segment (start 100.91 60.335) (end 101.025 60.45) (width 0.3) (layer "F.Cu") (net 5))
 (via (at 101.025 60.45) (size 0.6) (drill 0.3) (layers "F.Cu" "B.Cu") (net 5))
 (segment (start 101.025 60.45) (end 101.025 65.9) (width 0.3) (layer "B.Cu") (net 5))
 (segment (start 81.22 67.8) (end 79.78163 69.23837) (width 0.3) (layer "B.Cu") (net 5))
 (segment (start 99.125 67.8) (end 81.22 67.8) (width 0.3) (layer "B.Cu") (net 5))
 (segment (start 79.78163 69.23837) (end 79.78163 69.62) (width 0.3) (layer "B.Cu") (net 5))
 (segment (start 101.025 65.9) (end 99.125 67.8) (width 0.3) (layer "B.Cu") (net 5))
 (segment (start 95.83 55.325) (end 91.695 59.46) (width 0.3) (layer "F.Cu") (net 1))
 (segment (start 91.695 59.46) (end 79.4 59.46) (width 0.3) (layer "F.Cu") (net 1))
 (segment (start 89.280041 95.394959) (end 99.175 85.5) (width 0.3) (layer "F.Cu") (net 2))
 (segment (start 89.229138 95.394959) (end 89.280041 95.394959) (width 0.3) (layer "F.Cu") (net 2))
 (via (at 99.175 85.5) (size 0.6) (drill 0.3) (layers "F.Cu" "B.Cu") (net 2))
 (segment (start 86.3 65) (end 83.3 62) (width 0.3) (layer "B.Cu") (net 2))
 (segment (start 97.875 59.975) (end 97.875 62.325) (width 0.3) (layer "B.Cu") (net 2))
 (segment (start 86.3 65.05) (end 86.3 65) (width 0.3) (layer "B.Cu") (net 2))
 (segment (start 100.45 58.675) (end 99.175 58.675) (width 0.3) (layer "B.Cu") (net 2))
 (segment (start 107.8 76.875) (end 107.8 66.025) (width 0.3) (layer "B.Cu") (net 2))
 (segment (start 97.875 62.325) (end 95.15 65.05) (width 0.3) (layer "B.Cu") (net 2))
 (segment (start 107.8 66.025) (end 100.45 58.675) (width 0.3) (layer "B.Cu") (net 2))
 (segment (start 95.15 65.05) (end 86.3 65.05) (width 0.3) (layer "B.Cu") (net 2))
 (segment (start 99.175 58.675) (end 97.875 59.975) (width 0.3) (layer "B.Cu") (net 2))
 (segment (start 83.3 62) (end 79.4 62) (width 0.3) (layer "B.Cu") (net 2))
 (segment (start 99.175 85.5) (end 107.8 76.875) (width 0.3) (layer "B.Cu") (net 2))
 (segment (start 104.469138 97.530862) (end 103.375 98.625) (width 0.5) (layer "F.Cu") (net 15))
 (segment (start 104.469138 75.894138) (end 104.45 75.875) (width 0.5) (layer "F.Cu") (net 15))
 (segment (start 105.99 67.685) (end 105.925 67.75) (width 0.3) (layer "F.Cu") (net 15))
 (segment (start 104.469138 95.394959) (end 104.469138 75.894138) (width 0.5) (layer "F.Cu") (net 15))
 (segment (start 104.469138 95.394959) (end 104.469138 97.530862) (width 0.5) (layer "F.Cu") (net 15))
 (segment (start 105.99 55.325) (end 105.99 67.685) (width 0.5) (layer "F.Cu") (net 15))
 (segment (start 105.99 55.325) (end 105.975 55.34) (width 0.3) (layer "F.Cu") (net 15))
 (via (at 105.99 67.685) (size 0.6) (drill 0.3) (layers "F.Cu" "B.Cu") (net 15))
 (via (at 103.375 98.625) (size 0.6) (drill 0.3) (layers "F.Cu" "B.Cu") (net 15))
 (via (at 104.469138 75.894138) (size 0.6) (drill 0.3) (layers "F.Cu" "B.Cu") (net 15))
 (segment (start 104.45 69.225) (end 105.925 67.75) (width 0.5) (layer "B.Cu") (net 15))
 (segment (start 83.005 98.625) (end 79.4 95.02) (width 0.5) (layer "B.Cu") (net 15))
 (segment (start 104.45 75.875) (end 104.45 69.225) (width 0.5) (layer "B.Cu") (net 15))
 (segment (start 103.375 98.625) (end 83.005 98.625) (width 0.5) (layer "B.Cu") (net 15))
 (segment (start 92.425 62.05) (end 87.265108 62.05) (width 0.3) (layer "F.Cu") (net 7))
 (segment (start 82.7 74.225) (end 82.225 74.7) (width 0.3) (layer "F.Cu") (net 7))
 (segment (start 82.7 66.615108) (end 82.7 74.225) (width 0.3) (layer "F.Cu") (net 7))
 (segment (start 87.265108 62.05) (end 82.7 66.615108) (width 0.3) (layer "F.Cu") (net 7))
 (segment (start 82.225 74.7) (end 79.4 74.7) (width 0.3) (layer "F.Cu") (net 7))
 (via (at 92.425 62.05) (size 0.6) (drill 0.3) (layers "F.Cu" "B.Cu") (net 7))
 (segment (start 92.425 62.05) (end 93.275 61.2) (width 0.3) (layer "B.Cu") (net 7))
 (segment (start 93.275 55.555322) (end 93.29 55.555322) (width 0.3) (layer "B.Cu") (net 7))
 (segment (start 93.275 61.2) (end 93.275 55.555322) (width 0.3) (layer "B.Cu") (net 7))
 (segment (start 81.75 69.9) (end 81.75 66.15) (width 0.3) (layer "F.Cu") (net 6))
 (segment (start 81.75 66.15) (end 86.825 61.075) (width 0.3) (layer "F.Cu") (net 6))
 (segment (start 79.49 72.16) (end 81.75 69.9) (width 0.3) (layer "F.Cu") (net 6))
 (segment (start 79.4 72.16) (end 79.49 72.16) (width 0.3) (layer "F.Cu") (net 6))
 (via (at 86.825 61.075) (size 0.6) (drill 0.3) (layers "F.Cu" "B.Cu") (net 6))
 (segment (start 90.75 59.85) (end 90.75 55.325) (width 0.3) (layer "B.Cu") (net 6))
 (segment (start 87 60.9) (end 89.7 60.9) (width 0.3) (layer "B.Cu") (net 6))
 (segment (start 89.7 60.9) (end 90.75 59.85) (width 0.3) (layer "B.Cu") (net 6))
 (segment (start 86.825 61.075) (end 87 60.9) (width 0.3) (layer "B.Cu") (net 6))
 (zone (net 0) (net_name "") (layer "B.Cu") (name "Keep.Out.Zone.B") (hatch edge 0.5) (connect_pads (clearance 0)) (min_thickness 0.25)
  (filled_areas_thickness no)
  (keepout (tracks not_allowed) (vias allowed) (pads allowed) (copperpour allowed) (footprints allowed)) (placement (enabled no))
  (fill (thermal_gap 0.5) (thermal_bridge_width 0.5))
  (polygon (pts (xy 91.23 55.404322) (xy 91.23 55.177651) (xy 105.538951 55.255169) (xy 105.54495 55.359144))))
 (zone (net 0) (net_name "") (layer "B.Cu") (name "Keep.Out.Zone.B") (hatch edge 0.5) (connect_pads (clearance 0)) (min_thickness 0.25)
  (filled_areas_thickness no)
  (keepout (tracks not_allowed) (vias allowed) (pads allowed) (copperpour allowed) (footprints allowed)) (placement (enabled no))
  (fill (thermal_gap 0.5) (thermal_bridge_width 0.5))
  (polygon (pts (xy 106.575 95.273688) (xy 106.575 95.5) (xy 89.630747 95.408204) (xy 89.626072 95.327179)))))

